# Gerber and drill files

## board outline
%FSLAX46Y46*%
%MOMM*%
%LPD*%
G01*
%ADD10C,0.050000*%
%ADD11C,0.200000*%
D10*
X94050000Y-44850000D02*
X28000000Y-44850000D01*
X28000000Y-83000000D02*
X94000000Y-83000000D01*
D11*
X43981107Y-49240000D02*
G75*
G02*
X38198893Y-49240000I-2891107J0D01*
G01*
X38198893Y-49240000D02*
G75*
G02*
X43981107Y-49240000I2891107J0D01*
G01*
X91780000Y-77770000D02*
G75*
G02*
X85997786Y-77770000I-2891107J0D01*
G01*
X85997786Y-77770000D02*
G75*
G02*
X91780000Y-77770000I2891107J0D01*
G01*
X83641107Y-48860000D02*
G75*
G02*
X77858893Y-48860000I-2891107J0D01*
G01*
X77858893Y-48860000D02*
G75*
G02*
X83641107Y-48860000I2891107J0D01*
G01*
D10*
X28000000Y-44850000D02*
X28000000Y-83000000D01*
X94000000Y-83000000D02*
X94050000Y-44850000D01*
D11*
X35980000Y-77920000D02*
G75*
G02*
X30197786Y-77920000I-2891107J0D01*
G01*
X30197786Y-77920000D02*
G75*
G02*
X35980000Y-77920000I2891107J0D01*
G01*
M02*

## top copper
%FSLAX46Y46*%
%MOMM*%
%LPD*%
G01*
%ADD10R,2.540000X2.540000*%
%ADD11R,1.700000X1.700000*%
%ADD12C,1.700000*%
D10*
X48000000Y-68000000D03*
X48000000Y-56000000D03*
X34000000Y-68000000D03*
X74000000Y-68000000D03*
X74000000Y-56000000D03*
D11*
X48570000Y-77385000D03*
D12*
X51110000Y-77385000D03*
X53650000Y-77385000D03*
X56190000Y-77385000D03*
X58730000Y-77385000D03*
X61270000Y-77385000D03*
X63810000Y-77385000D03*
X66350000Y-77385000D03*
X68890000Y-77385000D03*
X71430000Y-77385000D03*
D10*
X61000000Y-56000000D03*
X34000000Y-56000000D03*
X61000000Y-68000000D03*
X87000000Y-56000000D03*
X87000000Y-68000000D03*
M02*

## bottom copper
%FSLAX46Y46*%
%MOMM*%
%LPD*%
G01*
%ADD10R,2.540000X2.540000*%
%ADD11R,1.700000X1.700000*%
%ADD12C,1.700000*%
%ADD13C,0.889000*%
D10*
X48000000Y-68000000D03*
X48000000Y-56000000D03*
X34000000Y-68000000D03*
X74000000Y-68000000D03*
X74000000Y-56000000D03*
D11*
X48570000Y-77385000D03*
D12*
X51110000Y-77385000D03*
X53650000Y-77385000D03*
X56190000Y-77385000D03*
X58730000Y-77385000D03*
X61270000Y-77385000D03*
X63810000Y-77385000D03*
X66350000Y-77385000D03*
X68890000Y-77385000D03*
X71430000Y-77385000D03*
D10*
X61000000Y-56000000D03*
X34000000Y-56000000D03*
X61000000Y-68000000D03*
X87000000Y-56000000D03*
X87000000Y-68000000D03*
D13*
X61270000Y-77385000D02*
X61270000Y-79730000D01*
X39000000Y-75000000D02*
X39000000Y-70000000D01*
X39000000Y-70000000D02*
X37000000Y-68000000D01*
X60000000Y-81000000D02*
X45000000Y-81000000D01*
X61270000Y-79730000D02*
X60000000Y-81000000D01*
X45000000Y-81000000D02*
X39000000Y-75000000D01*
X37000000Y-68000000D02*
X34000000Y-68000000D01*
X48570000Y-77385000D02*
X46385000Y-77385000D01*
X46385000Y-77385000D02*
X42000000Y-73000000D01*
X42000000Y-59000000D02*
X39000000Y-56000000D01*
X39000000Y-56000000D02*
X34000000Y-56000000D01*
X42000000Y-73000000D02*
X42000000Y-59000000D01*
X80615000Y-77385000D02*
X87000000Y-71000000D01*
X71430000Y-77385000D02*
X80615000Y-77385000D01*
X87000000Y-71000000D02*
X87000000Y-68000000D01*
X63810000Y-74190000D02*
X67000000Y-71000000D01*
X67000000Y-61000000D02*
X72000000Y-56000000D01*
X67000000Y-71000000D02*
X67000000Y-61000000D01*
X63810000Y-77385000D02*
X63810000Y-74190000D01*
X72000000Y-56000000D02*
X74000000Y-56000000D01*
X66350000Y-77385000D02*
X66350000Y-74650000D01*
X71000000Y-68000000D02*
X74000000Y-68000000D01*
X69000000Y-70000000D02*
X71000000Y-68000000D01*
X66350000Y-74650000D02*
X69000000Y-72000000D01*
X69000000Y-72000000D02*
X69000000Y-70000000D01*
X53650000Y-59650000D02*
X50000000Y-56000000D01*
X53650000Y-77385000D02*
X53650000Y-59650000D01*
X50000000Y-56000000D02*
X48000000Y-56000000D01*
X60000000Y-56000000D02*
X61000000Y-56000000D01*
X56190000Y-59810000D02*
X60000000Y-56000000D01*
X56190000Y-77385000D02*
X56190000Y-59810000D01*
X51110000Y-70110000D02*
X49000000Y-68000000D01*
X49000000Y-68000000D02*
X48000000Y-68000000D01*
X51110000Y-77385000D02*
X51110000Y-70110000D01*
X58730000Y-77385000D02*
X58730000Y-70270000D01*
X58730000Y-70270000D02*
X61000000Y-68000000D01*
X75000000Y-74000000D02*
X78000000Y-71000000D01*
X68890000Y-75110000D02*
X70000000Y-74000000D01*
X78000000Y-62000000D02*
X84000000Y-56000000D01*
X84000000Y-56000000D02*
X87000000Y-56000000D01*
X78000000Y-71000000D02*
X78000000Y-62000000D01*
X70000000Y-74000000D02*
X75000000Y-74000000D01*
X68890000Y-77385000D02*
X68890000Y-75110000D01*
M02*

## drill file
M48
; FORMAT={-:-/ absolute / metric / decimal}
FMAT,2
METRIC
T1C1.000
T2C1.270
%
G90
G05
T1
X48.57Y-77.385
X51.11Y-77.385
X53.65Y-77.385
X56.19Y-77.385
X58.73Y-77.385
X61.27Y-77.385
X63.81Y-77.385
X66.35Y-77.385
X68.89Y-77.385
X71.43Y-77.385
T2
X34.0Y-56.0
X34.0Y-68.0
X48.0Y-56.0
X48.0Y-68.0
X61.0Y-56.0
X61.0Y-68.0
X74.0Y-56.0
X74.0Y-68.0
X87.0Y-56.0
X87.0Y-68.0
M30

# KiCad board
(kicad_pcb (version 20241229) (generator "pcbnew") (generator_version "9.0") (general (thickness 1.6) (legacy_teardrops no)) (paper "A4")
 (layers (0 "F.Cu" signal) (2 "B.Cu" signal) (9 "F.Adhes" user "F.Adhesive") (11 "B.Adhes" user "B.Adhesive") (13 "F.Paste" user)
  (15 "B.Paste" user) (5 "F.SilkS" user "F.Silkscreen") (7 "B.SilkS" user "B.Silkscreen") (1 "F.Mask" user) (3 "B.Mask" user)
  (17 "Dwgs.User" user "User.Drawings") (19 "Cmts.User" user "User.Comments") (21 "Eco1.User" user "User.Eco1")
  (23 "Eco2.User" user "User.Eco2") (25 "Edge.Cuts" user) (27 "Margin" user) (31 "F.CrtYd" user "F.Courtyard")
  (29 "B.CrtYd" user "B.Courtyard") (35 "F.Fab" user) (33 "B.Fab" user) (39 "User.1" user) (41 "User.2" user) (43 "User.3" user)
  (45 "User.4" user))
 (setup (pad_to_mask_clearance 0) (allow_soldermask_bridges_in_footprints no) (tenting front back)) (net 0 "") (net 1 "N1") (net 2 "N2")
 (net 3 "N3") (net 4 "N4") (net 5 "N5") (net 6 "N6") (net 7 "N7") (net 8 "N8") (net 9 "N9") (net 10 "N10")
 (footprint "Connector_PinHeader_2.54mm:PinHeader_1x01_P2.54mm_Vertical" (layer "F.Cu") (at 48 68 180)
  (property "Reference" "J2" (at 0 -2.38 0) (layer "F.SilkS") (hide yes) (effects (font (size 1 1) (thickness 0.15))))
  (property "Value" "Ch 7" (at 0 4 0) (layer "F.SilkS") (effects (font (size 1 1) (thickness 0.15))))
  (pad "1" thru_hole rect (at 0 0 180) (size 2.54 2.54) (drill 1.27) (layers "*.Cu" "*.Mask") (remove_unused_layers no) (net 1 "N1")))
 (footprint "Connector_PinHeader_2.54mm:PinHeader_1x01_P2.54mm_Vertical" (layer "F.Cu") (at 48 56 180)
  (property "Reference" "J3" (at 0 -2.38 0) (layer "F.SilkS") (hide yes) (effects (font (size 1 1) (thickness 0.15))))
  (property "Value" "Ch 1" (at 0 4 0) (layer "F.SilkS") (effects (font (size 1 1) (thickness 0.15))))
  (pad "1" thru_hole rect (at 0 0 180) (size 2.54 2.54) (drill 1.27) (layers "*.Cu" "*.Mask") (remove_unused_layers no) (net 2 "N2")))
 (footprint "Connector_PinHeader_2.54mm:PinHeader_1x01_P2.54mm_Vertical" (layer "F.Cu") (at 34 68 180)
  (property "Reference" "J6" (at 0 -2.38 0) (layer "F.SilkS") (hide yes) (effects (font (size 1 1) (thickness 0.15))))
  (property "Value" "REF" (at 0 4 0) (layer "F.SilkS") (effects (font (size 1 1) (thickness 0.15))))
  (pad "1" thru_hole rect (at 0 0 180) (size 2.54 2.54) (drill 1.27) (layers "*.Cu" "*.Mask") (remove_unused_layers no) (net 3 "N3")))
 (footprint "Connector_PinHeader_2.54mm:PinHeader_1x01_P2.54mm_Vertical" (layer "F.Cu") (at 74 68 180)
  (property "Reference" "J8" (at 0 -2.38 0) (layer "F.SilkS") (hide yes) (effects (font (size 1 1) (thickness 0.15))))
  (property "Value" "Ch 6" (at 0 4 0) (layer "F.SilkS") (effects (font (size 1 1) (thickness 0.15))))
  (pad "1" thru_hole rect (at 0 0 180) (size 2.54 2.54) (drill 1.27) (layers "*.Cu" "*.Mask") (remove_unused_layers no) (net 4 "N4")))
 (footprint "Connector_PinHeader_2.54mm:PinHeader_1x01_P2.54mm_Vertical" (layer "F.Cu") (at 74 56 180)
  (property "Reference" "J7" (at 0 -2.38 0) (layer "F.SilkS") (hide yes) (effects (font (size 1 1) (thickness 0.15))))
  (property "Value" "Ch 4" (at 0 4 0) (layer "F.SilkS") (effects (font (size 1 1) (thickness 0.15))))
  (pad "1" thru_hole rect (at 0 0 180) (size 2.54 2.54) (drill 1.27) (layers "*.Cu" "*.Mask") (remove_unused_layers no) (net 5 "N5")))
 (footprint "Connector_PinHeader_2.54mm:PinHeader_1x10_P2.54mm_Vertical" (layer "F.Cu") (at 48.57 77.385 90)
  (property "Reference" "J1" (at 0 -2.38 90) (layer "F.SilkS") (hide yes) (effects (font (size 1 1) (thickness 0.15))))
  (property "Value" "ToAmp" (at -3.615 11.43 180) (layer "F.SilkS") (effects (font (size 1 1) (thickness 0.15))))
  (pad "1" thru_hole rect (at 0 0 90) (size 1.7 1.7) (drill 1) (layers "*.Cu" "*.Mask") (remove_unused_layers no) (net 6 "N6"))
  (pad "2" thru_hole circle (at 0 2.54 90) (size 1.7 1.7) (drill 1) (layers "*.Cu" "*.Mask") (remove_unused_layers no) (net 1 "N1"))
  (pad "3" thru_hole circle (at 0 5.08 90) (size 1.7 1.7) (drill 1) (layers "*.Cu" "*.Mask") (remove_unused_layers no) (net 2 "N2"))
  (pad "4" thru_hole circle (at 0 7.62 90) (size 1.7 1.7) (drill 1) (layers "*.Cu" "*.Mask") (remove_unused_layers no) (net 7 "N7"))
  (pad "5" thru_hole circle (at 0 10.16 90) (size 1.7 1.7) (drill 1) (layers "*.Cu" "*.Mask") (remove_unused_layers no) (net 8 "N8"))
  (pad "6" thru_hole circle (at 0 12.7 90) (size 1.7 1.7) (drill 1) (layers "*.Cu" "*.Mask") (remove_unused_layers no) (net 3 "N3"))
  (pad "7" thru_hole circle (at 0 15.24 90) (size 1.7 1.7) (drill 1) (layers "*.Cu" "*.Mask") (remove_unused_layers no) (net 5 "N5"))
  (pad "8" thru_hole circle (at 0 17.78 90) (size 1.7 1.7) (drill 1) (layers "*.Cu" "*.Mask") (remove_unused_layers no) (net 4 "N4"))
  (pad "9" thru_hole circle (at 0 20.32 90) (size 1.7 1.7) (drill 1) (layers "*.Cu" "*.Mask") (remove_unused_layers no) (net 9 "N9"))
  (pad "10" thru_hole circle (at 0 22.86 90) (size 1.7 1.7) (drill 1) (layers "*.Cu" "*.Mask") (remove_unused_layers no) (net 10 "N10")))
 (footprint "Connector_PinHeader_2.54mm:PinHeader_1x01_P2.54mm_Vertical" (layer "F.Cu") (at 61 56 180)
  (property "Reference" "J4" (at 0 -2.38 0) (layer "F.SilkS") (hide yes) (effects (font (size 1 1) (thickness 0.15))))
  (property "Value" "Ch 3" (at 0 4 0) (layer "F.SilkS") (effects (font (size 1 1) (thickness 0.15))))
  (pad "1" thru_hole rect (at 0 0 180) (size 2.54 2.54) (drill 1.27) (layers "*.Cu" "*.Mask") (remove_unused_layers no) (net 7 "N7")))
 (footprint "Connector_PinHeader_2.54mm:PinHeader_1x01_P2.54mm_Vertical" (layer "F.Cu") (at 34 56 180)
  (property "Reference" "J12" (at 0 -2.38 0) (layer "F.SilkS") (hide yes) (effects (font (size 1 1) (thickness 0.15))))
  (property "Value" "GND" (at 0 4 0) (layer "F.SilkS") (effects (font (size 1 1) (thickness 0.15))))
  (pad "1" thru_hole rect (at 0 0 180) (size 2.54 2.54) (drill 1.27) (layers "*.Cu" "*.Mask") (remove_unused_layers no) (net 6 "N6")))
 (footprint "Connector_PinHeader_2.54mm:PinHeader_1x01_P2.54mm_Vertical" (layer "F.Cu") (at 61 68 180)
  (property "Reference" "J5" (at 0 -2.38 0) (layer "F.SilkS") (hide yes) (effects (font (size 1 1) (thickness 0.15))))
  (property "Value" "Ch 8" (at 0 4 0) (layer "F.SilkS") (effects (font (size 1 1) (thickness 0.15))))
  (pad "1" thru_hole rect (at 0 0 180) (size 2.54 2.54) (drill 1.27) (layers "*.Cu" "*.Mask") (remove_unused_layers no) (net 8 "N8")))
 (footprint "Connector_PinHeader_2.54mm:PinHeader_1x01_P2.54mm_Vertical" (layer "F.Cu") (at 87 56 180)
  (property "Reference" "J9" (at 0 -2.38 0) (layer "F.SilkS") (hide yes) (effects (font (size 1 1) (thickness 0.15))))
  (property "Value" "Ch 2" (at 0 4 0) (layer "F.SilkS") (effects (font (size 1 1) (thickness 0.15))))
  (pad "1" thru_hole rect (at 0 0 180) (size 2.54 2.54) (drill 1.27) (layers "*.Cu" "*.Mask") (remove_unused_layers no) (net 9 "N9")))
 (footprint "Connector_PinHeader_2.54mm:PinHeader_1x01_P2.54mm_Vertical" (layer "F.Cu") (at 87 68 180)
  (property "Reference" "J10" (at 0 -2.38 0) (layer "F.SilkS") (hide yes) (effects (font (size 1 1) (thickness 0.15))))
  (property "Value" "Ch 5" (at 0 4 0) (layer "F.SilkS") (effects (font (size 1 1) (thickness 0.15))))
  (pad "1" thru_hole rect (at 0 0 180) (size 2.54 2.54) (drill 1.27) (layers "*.Cu" "*.Mask") (remove_unused_layers no) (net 10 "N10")))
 (gr_line (start 94.05 44.85) (end 28 44.85) (stroke (width 0.05) (type default)) (layer "Edge.Cuts"))
 (gr_line (start 28 83) (end 94 83) (stroke (width 0.05) (type default)) (layer "Edge.Cuts"))
 (gr_circle (center 41.09 49.24) (end 43.32 51.08) (stroke (width 0.2) (type solid)) (fill no) (layer "Edge.Cuts"))
 (gr_circle (center 88.888893 77.77) (end 91.118893 79.61) (stroke (width 0.2) (type solid)) (fill no) (layer "Edge.Cuts"))
 (gr_circle (center 80.75 48.86) (end 82.98 50.7) (stroke (width 0.2) (type solid)) (fill no) (layer "Edge.Cuts"))
 (gr_line (start 28 44.85) (end 28 83) (stroke (width 0.05) (type default)) (layer "Edge.Cuts"))
 (gr_line (start 94 83) (end 94.05 44.85) (stroke (width 0.05) (type default)) (layer "Edge.Cuts"))
 (gr_circle (center 33.088893 77.92) (end 35.318893 79.76) (stroke (width 0.2) (type solid)) (fill no) (layer "Edge.Cuts"))
 (segment (start 61.27 77.385) (end 61.27 79.73) (width 0.889) (layer "B.Cu") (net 3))
 (segment (start 39 75) (end 39 70) (width 0.889) (layer "B.Cu") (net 3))
 (segment (start 39 70) (end 37 68) (width 0.889) (layer "B.Cu") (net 3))
 (segment (start 60 81) (end 45 81) (width 0.889) (layer "B.Cu") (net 3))
 (segment (start 61.27 79.73) (end 60 81) (width 0.889) (layer "B.Cu") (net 3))
 (segment (start 45 81) (end 39 75) (width 0.889) (layer "B.Cu") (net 3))
 (segment (start 37 68) (end 34 68) (width 0.889) (layer "B.Cu") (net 3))
 (segment (start 48.57 77.385) (end 46.385 77.385) (width 0.889) (layer "B.Cu") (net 6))
 (segment (start 46.385 77.385) (end 42 73) (width 0.889) (layer "B.Cu") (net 6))
 (segment (start 42 59) (end 39 56) (width 0.889) (layer "B.Cu") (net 6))
 (segment (start 39 56) (end 34 56) (width 0.889) (layer "B.Cu") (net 6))
 (segment (start 42 73) (end 42 59) (width 0.889) (layer "B.Cu") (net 6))
 (segment (start 80.615 77.385) (end 87 71) (width 0.889) (layer "B.Cu") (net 10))
 (segment (start 71.43 77.385) (end 80.615 77.385) (width 0.889) (layer "B.Cu") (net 10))
 (segment (start 87 71) (end 87 68) (width 0.889) (layer "B.Cu") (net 10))
 (segment (start 63.81 74.19) (end 67 71) (width 0.889) (layer "B.Cu") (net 5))
 (segment (start 67 61) (end 72 56) (width 0.889) (layer "B.Cu") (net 5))
 (segment (start 67 71) (end 67 61) (width 0.889) (layer "B.Cu") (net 5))
 (segment (start 63.81 77.385) (end 63.81 74.19) (width 0.889) (layer "B.Cu") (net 5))
 (segment (start 72 56) (end 74 56) (width 0.889) (layer "B.Cu") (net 5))
 (segment (start 66.35 77.385) (end 66.35 74.65) (width 0.889) (layer "B.Cu") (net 4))
 (segment (start 71 68) (end 74 68) (width 0.889) (layer "B.Cu") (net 4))
 (segment (start 69 70) (end 71 68) (width 0.889) (layer "B.Cu") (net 4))
 (segment (start 66.35 74.65) (end 69 72) (width 0.889) (layer "B.Cu") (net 4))
 (segment (start 69 72) (end 69 70) (width 0.889) (layer "B.Cu") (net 4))
 (segment (start 53.65 59.65) (end 50 56) (width 0.889) (layer "B.Cu") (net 2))
 (segment (start 53.65 77.385) (end 53.65 59.65) (width 0.889) (layer "B.Cu") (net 2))
 (segment (start 50 56) (end 48 56) (width 0.889) (layer "B.Cu") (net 2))
 (segment (start 60 56) (end 61 56) (width 0.889) (layer "B.Cu") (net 7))
 (segment (start 56.19 59.81) (end 60 56) (width 0.889) (layer "B.Cu") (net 7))
 (segment (start 56.19 77.385) (end 56.19 59.81) (width 0.889) (layer "B.Cu") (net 7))
 (segment (start 51.11 70.11) (end 49 68) (width 0.889) (layer "B.Cu") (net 1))
 (segment (start 49 68) (end 48 68) (width 0.889) (layer "B.Cu") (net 1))
 (segment (start 51.11 77.385) (end 51.11 70.11) (width 0.889) (layer "B.Cu") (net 1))
 (segment (start 58.73 77.385) (end 58.73 70.27) (width 0.889) (layer "B.Cu") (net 8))
 (segment (start 58.73 70.27) (end 61 68) (width 0.889) (layer "B.Cu") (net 8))
 (segment (start 75 74) (end 78 71) (width 0.889) (layer "B.Cu") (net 9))
 (segment (start 68.89 75.11) (end 70 74) (width 0.889) (layer "B.Cu") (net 9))
 (segment (start 78 62) (end 84 56) (width 0.889) (layer "B.Cu") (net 9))
 (segment (start 84 56) (end 87 56) (width 0.889) (layer "B.Cu") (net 9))
 (segment (start 78 71) (end 78 62) (width 0.889) (layer "B.Cu") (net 9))
 (segment (start 70 74) (end 75 74) (width 0.889) (layer "B.Cu") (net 9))
 (segment (start 68.89 77.385) (end 68.89 75.11) (width 0.889) (layer "B.Cu") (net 9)))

